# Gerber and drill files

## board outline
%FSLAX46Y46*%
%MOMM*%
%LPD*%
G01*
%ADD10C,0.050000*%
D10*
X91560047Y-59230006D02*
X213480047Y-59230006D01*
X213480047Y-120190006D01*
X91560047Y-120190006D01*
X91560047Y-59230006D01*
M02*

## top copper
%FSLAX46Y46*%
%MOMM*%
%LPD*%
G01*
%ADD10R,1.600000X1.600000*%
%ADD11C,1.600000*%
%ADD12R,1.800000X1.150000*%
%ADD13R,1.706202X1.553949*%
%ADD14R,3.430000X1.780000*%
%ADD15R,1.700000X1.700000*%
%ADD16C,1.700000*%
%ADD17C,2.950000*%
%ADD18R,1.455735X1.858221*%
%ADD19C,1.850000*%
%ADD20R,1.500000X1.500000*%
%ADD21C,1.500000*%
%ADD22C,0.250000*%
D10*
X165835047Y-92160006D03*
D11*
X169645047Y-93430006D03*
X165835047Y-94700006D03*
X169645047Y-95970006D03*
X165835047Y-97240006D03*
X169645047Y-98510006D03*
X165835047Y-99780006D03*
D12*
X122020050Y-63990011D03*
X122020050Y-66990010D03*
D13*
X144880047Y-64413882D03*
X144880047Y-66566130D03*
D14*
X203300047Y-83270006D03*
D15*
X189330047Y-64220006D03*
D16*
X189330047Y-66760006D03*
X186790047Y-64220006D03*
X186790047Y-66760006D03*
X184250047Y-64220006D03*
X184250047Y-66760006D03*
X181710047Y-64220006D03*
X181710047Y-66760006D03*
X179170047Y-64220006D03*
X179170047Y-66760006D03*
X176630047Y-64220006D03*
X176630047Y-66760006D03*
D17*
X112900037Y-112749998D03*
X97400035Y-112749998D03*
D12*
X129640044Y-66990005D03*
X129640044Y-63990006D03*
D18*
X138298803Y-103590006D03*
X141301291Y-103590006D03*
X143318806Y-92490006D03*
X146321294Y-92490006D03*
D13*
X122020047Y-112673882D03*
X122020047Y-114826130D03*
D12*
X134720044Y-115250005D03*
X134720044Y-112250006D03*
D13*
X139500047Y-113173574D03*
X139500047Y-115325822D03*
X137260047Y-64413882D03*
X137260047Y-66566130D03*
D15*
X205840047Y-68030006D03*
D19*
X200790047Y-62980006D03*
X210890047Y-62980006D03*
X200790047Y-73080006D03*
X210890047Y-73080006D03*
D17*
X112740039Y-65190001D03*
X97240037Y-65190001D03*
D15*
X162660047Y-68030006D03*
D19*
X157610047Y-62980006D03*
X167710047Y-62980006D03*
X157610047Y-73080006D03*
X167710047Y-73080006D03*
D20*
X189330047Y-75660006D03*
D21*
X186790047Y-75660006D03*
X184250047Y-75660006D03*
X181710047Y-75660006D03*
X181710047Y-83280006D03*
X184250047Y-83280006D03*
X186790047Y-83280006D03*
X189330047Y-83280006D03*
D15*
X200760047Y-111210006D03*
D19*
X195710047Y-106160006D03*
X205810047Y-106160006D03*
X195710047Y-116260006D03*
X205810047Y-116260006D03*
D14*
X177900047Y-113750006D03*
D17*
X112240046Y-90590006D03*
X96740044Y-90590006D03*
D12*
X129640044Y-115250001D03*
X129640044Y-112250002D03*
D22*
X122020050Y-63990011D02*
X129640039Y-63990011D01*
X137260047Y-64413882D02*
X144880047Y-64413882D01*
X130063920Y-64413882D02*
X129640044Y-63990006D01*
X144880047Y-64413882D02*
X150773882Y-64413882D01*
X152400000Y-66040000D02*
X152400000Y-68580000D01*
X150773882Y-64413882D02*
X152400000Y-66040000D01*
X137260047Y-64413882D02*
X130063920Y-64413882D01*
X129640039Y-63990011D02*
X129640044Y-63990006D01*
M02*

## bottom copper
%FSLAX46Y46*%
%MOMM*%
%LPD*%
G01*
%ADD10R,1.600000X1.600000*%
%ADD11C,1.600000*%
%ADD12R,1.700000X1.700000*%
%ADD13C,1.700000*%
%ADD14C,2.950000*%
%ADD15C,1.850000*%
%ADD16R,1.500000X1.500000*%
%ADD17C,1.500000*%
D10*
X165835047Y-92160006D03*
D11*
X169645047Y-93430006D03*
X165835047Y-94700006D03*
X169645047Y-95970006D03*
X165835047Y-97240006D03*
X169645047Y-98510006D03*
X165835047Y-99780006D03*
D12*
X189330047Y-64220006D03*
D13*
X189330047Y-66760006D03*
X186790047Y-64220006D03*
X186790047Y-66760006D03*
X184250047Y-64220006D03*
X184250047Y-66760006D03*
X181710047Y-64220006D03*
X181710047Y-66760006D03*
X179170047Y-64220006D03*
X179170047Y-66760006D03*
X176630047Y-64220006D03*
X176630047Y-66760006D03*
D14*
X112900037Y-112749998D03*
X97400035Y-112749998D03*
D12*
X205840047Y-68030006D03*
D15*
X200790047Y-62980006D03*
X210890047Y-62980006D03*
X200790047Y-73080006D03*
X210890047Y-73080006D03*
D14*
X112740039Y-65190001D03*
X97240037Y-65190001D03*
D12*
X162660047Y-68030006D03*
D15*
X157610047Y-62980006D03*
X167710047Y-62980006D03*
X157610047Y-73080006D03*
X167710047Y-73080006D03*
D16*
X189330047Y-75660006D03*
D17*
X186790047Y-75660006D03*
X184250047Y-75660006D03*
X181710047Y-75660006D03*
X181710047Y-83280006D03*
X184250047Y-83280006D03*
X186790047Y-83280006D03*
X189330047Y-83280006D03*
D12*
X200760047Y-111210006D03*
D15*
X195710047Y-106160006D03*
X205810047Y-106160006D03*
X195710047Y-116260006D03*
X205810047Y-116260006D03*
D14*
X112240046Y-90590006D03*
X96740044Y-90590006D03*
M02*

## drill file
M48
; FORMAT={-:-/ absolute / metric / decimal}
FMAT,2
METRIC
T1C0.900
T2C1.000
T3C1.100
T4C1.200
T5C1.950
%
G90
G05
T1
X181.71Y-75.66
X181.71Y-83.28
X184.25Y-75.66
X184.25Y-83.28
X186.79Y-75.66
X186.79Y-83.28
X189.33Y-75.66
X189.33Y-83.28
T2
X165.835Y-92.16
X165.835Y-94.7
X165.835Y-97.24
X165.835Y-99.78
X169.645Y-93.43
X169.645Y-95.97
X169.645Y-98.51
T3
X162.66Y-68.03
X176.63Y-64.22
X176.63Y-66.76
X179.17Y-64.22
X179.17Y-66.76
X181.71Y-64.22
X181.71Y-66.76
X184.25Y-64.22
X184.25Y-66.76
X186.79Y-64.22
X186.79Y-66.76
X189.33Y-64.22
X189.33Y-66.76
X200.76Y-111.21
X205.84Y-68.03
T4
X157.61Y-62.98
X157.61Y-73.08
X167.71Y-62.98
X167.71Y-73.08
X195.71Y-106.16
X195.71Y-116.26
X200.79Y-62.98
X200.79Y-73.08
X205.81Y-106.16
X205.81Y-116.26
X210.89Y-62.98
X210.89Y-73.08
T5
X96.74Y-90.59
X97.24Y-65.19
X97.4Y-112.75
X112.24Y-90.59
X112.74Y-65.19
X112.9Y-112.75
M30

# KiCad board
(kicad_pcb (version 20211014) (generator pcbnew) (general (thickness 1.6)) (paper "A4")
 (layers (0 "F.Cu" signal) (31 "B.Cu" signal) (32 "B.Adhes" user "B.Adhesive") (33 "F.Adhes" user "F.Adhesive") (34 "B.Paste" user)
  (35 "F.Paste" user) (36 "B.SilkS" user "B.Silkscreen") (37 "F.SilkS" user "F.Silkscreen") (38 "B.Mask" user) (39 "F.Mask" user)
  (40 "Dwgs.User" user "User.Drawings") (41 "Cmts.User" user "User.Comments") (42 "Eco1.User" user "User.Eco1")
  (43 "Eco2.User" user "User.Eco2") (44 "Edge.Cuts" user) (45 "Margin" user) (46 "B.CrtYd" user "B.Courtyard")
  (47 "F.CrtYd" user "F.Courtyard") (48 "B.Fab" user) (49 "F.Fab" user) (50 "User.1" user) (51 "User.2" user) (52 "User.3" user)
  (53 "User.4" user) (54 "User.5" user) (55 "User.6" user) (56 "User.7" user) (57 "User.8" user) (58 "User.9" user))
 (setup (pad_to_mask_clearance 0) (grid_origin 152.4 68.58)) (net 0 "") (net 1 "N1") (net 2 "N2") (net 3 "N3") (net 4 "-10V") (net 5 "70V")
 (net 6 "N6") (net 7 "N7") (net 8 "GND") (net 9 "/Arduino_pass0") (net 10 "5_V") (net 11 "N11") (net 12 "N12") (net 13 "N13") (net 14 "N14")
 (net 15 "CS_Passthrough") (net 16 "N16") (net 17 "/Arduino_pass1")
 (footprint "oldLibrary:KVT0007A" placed (layer "F.Cu") (at 167.740047 95.970006)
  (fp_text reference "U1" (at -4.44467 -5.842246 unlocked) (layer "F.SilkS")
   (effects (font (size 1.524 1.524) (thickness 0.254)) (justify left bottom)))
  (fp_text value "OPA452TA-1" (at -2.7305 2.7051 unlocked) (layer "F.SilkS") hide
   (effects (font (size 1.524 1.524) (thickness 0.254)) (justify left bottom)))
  (pad "1" thru_hole rect (at -1.905 -3.81) (size 1.6 1.6) (drill 1) (layers *.Cu *.Mask) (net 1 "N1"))
  (pad "2" thru_hole circle (at 1.905 -2.54) (size 1.6 1.6) (drill 1) (layers *.Cu *.Mask) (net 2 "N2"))
  (pad "3" thru_hole circle (at -1.905 -1.27) (size 1.6 1.6) (drill 1) (layers *.Cu *.Mask) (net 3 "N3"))
  (pad "4" thru_hole circle (at 1.905 0) (size 1.6 1.6) (drill 1) (layers *.Cu *.Mask) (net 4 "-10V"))
  (pad "5" thru_hole circle (at -1.905 1.27) (size 1.6 1.6) (drill 1) (layers *.Cu *.Mask) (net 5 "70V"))
  (pad "6" thru_hole circle (at 1.905 2.54) (size 1.6 1.6) (drill 1) (layers *.Cu *.Mask) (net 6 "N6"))
  (pad "7" thru_hole circle (at -1.905 3.81) (size 1.6 1.6) (drill 1) (layers *.Cu *.Mask) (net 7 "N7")))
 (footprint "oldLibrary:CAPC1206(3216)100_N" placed (layer "F.Cu") (at 122.020047 65.49001 -90)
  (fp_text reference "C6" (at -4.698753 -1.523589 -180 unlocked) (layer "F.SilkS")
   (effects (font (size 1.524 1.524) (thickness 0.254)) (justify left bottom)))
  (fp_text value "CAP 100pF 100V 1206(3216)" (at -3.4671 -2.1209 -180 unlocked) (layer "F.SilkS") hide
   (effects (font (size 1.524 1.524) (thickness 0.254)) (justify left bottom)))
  (pad "1" smd rect (at -1.499999 -0.000003) (size 1.8 1.15) (layers "F.Cu" "F.Paste" "F.Mask") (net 4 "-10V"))
  (pad "2" smd rect (at 1.5 -0.000003) (size 1.8 1.15) (layers "F.Cu" "F.Paste" "F.Mask") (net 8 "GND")))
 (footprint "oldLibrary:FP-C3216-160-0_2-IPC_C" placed (layer "F.Cu") (at 144.880047 65.490006 -90)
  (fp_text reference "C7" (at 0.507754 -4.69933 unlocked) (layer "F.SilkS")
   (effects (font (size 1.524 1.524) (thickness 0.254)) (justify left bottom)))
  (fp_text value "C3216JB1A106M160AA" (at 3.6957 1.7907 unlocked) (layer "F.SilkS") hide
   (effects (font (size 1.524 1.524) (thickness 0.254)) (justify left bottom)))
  (pad "1" smd rect (at -1.076124 0 270) (size 1.553949 1.706202) (layers "F.Cu" "F.Paste" "F.Mask") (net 4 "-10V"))
  (pad "2" smd rect (at 1.076124 0 270) (size 1.553949 1.706202) (layers "F.Cu" "F.Paste" "F.Mask") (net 8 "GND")))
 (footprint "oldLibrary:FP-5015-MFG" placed (layer "F.Cu") (at 203.300047 83.270006)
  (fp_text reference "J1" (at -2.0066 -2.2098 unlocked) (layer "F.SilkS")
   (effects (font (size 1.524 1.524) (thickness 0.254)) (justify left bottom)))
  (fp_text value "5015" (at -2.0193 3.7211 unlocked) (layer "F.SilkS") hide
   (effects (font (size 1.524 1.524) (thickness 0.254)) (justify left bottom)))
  (pad "1" smd rect (at 0 0) (size 3.43 1.78) (layers "F.Cu" "F.Paste" "F.Mask") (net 2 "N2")))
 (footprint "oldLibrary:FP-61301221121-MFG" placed (layer "F.Cu") (at 182.980047 65.490006 180)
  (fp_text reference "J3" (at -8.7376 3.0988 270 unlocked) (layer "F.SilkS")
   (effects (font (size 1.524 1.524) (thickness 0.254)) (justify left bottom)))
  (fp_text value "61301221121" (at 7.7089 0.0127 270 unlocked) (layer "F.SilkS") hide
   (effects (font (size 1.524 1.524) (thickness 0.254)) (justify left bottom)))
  (pad "1" thru_hole rect (at -6.35 1.27 180) (size 1.7 1.7) (drill 1.1) (layers *.Cu *.Mask) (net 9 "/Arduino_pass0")
   (solder_paste_margin -1000))
  (pad "2" thru_hole circle (at -6.35 -1.27 180) (size 1.7 1.7) (drill 1.1) (layers *.Cu *.Mask) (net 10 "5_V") (solder_paste_margin -1000))
  (pad "3" thru_hole circle (at -3.81 1.27 180) (size 1.7 1.7) (drill 1.1) (layers *.Cu *.Mask) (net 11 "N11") (solder_paste_margin -1000))
  (pad "4" thru_hole circle (at -3.81 -1.27 180) (size 1.7 1.7) (drill 1.1) (layers *.Cu *.Mask) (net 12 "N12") (solder_paste_margin -1000))
  (pad "5" thru_hole circle (at -1.27 1.27 180) (size 1.7 1.7) (drill 1.1) (layers *.Cu *.Mask) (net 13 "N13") (solder_paste_margin -1000))
  (pad "6" thru_hole circle (at -1.27 -1.27 180) (size 1.7 1.7) (drill 1.1) (layers *.Cu *.Mask) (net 13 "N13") (solder_paste_margin -1000))
  (pad "7" thru_hole circle (at 1.27 1.27 180) (size 1.7 1.7) (drill 1.1) (layers *.Cu *.Mask) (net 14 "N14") (solder_paste_margin -1000))
  (pad "8" thru_hole circle (at 1.27 -1.27 180) (size 1.7 1.7) (drill 1.1) (layers *.Cu *.Mask) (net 14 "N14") (solder_paste_margin -1000))
  (pad "9" thru_hole circle (at 3.81 1.27 180) (size 1.7 1.7) (drill 1.1) (layers *.Cu *.Mask) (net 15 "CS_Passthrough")
   (solder_paste_margin -1000))
  (pad "10" thru_hole circle (at 3.81 -1.27 180) (size 1.7 1.7) (drill 1.1) (layers *.Cu *.Mask) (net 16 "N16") (solder_paste_margin -1000))
  (pad "11" thru_hole circle (at 6.35 1.27 180) (size 1.7 1.7) (drill 1.1) (layers *.Cu *.Mask) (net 15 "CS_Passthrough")
   (solder_paste_margin -1000))
  (pad "12" thru_hole circle (at 6.35 -1.27 180) (size 1.7 1.7) (drill 1.1) (layers *.Cu *.Mask) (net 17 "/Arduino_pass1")
   (solder_paste_margin -1000)))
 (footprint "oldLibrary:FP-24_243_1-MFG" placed (layer "F.Cu") (at 104.400037 113.049998)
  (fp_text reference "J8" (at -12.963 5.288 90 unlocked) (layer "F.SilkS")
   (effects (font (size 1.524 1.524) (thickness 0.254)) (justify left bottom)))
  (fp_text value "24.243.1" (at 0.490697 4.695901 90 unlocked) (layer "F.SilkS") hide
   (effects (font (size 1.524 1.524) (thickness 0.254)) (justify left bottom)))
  (pad "1" thru_hole circle (at 8.5 -0.3) (size 2.95 2.95) (drill 1.95) (layers *.Cu *.Mask) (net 8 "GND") (solder_paste_margin -1000))
  (pad "1" thru_hole circle (at -7.000002 -0.3) (size 2.95 2.95) (drill 1.95) (layers *.Cu *.Mask) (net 8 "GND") (solder_paste_margin -1000)))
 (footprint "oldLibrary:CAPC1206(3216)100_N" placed (layer "F.Cu") (at 129.640047 65.490006 90)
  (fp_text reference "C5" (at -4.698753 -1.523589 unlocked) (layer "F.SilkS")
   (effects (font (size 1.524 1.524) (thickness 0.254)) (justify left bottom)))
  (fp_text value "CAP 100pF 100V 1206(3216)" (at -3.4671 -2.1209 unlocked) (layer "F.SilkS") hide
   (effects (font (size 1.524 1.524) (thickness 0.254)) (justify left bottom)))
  (pad "1" smd rect (at -1.499999 -0.000003 180) (size 1.8 1.15) (layers "F.Cu" "F.Paste" "F.Mask") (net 8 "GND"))
  (pad "2" smd rect (at 1.5 -0.000003 180) (size 1.8 1.15) (layers "F.Cu" "F.Paste" "F.Mask") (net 4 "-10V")))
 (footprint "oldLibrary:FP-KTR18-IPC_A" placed (layer "F.Cu") (at 139.800047 103.590006)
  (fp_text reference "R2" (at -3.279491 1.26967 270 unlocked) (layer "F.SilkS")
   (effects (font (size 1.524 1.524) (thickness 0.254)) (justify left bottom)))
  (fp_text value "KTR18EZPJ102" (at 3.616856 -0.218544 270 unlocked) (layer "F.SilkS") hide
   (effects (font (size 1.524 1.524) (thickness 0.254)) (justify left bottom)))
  (pad "1" smd rect (at -1.501244 0 180) (size 1.455735 1.858221) (layers "F.Cu" "F.Paste" "F.Mask") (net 8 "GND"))
  (pad "2" smd rect (at 1.501244 0 180) (size 1.455735 1.858221) (layers "F.Cu" "F.Paste" "F.Mask") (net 1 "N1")))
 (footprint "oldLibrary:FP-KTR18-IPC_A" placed (layer "F.Cu") (at 144.82005 92.490006)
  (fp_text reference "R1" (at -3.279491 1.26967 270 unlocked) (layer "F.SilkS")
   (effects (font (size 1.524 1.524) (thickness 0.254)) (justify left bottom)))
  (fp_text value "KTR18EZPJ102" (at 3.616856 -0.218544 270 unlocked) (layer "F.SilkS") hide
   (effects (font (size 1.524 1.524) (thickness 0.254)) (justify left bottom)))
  (pad "1" smd rect (at -1.501244 0 180) (size 1.455735 1.858221) (layers "F.Cu" "F.Paste" "F.Mask") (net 1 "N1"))
  (pad "2" smd rect (at 1.501244 0 180) (size 1.455735 1.858221) (layers "F.Cu" "F.Paste" "F.Mask") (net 6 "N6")))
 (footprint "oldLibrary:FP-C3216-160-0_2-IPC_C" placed (layer "F.Cu") (at 122.020047 113.750006 -90)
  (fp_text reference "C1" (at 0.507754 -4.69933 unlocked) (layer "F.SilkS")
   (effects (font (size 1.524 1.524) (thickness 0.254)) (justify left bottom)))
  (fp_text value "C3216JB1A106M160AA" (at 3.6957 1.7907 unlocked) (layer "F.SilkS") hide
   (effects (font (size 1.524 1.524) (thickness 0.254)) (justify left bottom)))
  (pad "1" smd rect (at -1.076124 0 270) (size 1.553949 1.706202) (layers "F.Cu" "F.Paste" "F.Mask") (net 5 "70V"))
  (pad "2" smd rect (at 1.076124 0 270) (size 1.553949 1.706202) (layers "F.Cu" "F.Paste" "F.Mask") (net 8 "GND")))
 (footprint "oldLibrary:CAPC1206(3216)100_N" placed (layer "F.Cu") (at 134.720047 113.750006 90)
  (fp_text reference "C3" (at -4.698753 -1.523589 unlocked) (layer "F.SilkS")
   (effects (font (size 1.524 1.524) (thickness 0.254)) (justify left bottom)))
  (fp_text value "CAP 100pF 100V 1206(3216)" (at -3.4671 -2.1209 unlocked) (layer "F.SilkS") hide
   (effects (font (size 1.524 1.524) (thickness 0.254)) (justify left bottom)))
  (pad "1" smd rect (at -1.499999 -0.000003 180) (size 1.8 1.15) (layers "F.Cu" "F.Paste" "F.Mask") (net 8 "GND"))
  (pad "2" smd rect (at 1.5 -0.000003 180) (size 1.8 1.15) (layers "F.Cu" "F.Paste" "F.Mask") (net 5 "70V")))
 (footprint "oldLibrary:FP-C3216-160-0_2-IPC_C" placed (layer "F.Cu") (at 139.500047 114.249698 -90)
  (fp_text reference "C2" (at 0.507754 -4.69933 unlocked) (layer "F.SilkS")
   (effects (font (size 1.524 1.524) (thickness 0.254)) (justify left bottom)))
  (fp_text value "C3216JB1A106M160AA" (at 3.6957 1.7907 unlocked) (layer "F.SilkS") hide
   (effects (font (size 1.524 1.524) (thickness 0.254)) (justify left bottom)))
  (pad "1" smd rect (at -1.076124 0 270) (size 1.553949 1.706202) (layers "F.Cu" "F.Paste" "F.Mask") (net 5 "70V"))
  (pad "2" smd rect (at 1.076124 0 270) (size 1.553949 1.706202) (layers "F.Cu" "F.Paste" "F.Mask") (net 8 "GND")))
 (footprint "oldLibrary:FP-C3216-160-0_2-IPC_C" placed (layer "F.Cu") (at 137.260047 65.490006 -90)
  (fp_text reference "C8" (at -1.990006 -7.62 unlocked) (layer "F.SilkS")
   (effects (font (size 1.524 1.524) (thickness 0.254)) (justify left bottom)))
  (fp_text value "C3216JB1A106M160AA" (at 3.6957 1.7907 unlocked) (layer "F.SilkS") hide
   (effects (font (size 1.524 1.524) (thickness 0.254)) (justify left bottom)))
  (pad "1" smd rect (at -1.076124 0 270) (size 1.553949 1.706202) (layers "F.Cu" "F.Paste" "F.Mask") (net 4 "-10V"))
  (pad "2" smd rect (at 1.076124 0 270) (size 1.553949 1.706202) (layers "F.Cu" "F.Paste" "F.Mask") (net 8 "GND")))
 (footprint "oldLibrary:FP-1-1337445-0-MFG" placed (layer "F.Cu") (at 205.840047 68.030006)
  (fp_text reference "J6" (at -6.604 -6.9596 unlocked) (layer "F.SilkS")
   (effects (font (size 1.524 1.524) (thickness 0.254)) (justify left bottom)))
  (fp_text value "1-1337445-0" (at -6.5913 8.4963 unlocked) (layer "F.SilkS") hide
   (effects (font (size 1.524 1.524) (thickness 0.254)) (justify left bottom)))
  (pad "1" thru_hole rect (at 0 0) (size 1.7 1.7) (drill 1.1) (layers *.Cu *.Mask) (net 9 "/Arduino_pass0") (solder_paste_margin -1000))
  (pad "2" thru_hole circle (at -5.05 -5.05) (size 1.85 1.85) (drill 1.2) (layers *.Cu *.Mask) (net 8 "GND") (solder_paste_margin -1000))
  (pad "3" thru_hole circle (at 5.05 -5.05) (size 1.85 1.85) (drill 1.2) (layers *.Cu *.Mask) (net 8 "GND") (solder_paste_margin -1000))
  (pad "4" thru_hole circle (at -5.05 5.05) (size 1.85 1.85) (drill 1.2) (layers *.Cu *.Mask) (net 8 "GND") (solder_paste_margin -1000))
  (pad "5" thru_hole circle (at 5.05 5.05) (size 1.85 1.85) (drill 1.2) (layers *.Cu *.Mask) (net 8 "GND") (solder_paste_margin -1000)))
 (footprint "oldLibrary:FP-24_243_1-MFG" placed (layer "F.Cu") (at 104.240039 65.490001)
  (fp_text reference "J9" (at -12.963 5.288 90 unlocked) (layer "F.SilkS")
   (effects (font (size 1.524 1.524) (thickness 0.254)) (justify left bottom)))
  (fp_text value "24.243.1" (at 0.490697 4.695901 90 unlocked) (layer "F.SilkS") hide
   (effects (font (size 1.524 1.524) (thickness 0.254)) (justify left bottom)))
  (pad "1" thru_hole circle (at 8.5 -0.3) (size 2.95 2.95) (drill 1.95) (layers *.Cu *.Mask) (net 4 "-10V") (solder_paste_margin -1000))
  (pad "1" thru_hole circle (at -7.000002 -0.3) (size 2.95 2.95) (drill 1.95) (layers *.Cu *.Mask) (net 4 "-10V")
   (solder_paste_margin -1000)))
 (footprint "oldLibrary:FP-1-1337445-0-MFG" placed (layer "F.Cu") (at 162.660047 68.030006)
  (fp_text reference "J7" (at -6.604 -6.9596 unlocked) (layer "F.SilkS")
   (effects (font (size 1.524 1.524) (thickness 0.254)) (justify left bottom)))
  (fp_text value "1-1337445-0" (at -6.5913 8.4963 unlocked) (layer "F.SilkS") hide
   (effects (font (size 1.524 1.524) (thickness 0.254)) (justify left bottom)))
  (pad "1" thru_hole rect (at 0 0) (size 1.7 1.7) (drill 1.1) (layers *.Cu *.Mask) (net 17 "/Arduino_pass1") (solder_paste_margin -1000))
  (pad "2" thru_hole circle (at -5.05 -5.05) (size 1.85 1.85) (drill 1.2) (layers *.Cu *.Mask) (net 8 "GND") (solder_paste_margin -1000))
  (pad "3" thru_hole circle (at 5.05 -5.05) (size 1.85 1.85) (drill 1.2) (layers *.Cu *.Mask) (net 8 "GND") (solder_paste_margin -1000))
  (pad "4" thru_hole circle (at -5.05 5.05) (size 1.85 1.85) (drill 1.2) (layers *.Cu *.Mask) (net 8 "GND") (solder_paste_margin -1000))
  (pad "5" thru_hole circle (at 5.05 5.05) (size 1.85 1.85) (drill 1.2) (layers *.Cu *.Mask) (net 8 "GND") (solder_paste_margin -1000)))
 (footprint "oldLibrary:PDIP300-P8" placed (layer "F.Cu") (at 185.520047 79.470006 -90)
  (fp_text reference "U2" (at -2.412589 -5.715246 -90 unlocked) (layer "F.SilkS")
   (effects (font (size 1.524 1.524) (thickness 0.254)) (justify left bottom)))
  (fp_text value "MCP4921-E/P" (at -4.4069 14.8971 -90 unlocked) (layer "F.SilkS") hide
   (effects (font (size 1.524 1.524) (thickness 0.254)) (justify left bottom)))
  (pad "1" thru_hole rect (at -3.81 -3.81 270) (size 1.5 1.5) (drill 0.9) (layers *.Cu *.Mask) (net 10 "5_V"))
  (pad "2" thru_hole circle (at -3.81 -1.27 270) (size 1.5 1.5) (drill 0.9) (layers *.Cu *.Mask) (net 12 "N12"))
  (pad "3" thru_hole circle (at -3.81 1.27 270) (size 1.5 1.5) (drill 0.9) (layers *.Cu *.Mask) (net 13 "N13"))
  (pad "4" thru_hole circle (at -3.81 3.81 270) (size 1.5 1.5) (drill 0.9) (layers *.Cu *.Mask) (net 14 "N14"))
  (pad "5" thru_hole circle (at 3.81 3.81 270) (size 1.5 1.5) (drill 0.9) (layers *.Cu *.Mask) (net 16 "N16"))
  (pad "6" thru_hole circle (at 3.81 1.27 270) (size 1.5 1.5) (drill 0.9) (layers *.Cu *.Mask) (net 10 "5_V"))
  (pad "7" thru_hole circle (at 3.81 -1.27 270) (size 1.5 1.5) (drill 0.9) (layers *.Cu *.Mask) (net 8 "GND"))
  (pad "8" thru_hole circle (at 3.81 -3.81 270) (size 1.5 1.5) (drill 0.9) (layers *.Cu *.Mask) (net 2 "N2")))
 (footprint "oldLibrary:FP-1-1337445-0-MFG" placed (layer "F.Cu") (at 200.760047 111.210006)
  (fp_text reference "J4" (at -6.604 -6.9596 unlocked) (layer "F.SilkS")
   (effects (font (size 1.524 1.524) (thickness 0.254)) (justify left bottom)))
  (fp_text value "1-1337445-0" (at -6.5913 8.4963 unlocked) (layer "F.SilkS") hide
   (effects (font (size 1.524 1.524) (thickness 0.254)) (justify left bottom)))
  (pad "1" thru_hole rect (at 0 0) (size 1.7 1.7) (drill 1.1) (layers *.Cu *.Mask) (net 6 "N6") (solder_paste_margin -1000))
  (pad "2" thru_hole circle (at -5.05 -5.05) (size 1.85 1.85) (drill 1.2) (layers *.Cu *.Mask) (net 8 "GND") (solder_paste_margin -1000))
  (pad "3" thru_hole circle (at 5.05 -5.05) (size 1.85 1.85) (drill 1.2) (layers *.Cu *.Mask) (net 8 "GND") (solder_paste_margin -1000))
  (pad "4" thru_hole circle (at -5.05 5.05) (size 1.85 1.85) (drill 1.2) (layers *.Cu *.Mask) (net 8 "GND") (solder_paste_margin -1000))
  (pad "5" thru_hole circle (at 5.05 5.05) (size 1.85 1.85) (drill 1.2) (layers *.Cu *.Mask) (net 8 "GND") (solder_paste_margin -1000)))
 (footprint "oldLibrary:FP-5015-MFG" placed (layer "F.Cu") (at 177.900047 113.750006)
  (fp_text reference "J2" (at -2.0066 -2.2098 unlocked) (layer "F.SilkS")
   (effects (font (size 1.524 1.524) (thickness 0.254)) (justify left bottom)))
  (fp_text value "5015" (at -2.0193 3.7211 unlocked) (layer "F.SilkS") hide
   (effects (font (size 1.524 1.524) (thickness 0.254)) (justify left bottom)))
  (pad "1" smd rect (at 0 0) (size 3.43 1.78) (layers "F.Cu" "F.Paste" "F.Mask") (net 6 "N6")))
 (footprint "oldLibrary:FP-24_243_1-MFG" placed (layer "F.Cu") (at 103.740046 90.890006)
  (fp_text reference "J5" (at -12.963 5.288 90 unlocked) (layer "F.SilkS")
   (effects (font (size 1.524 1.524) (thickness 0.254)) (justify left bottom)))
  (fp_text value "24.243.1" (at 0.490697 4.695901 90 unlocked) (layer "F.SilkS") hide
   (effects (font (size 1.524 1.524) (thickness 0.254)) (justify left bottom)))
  (pad "1" thru_hole circle (at 8.5 -0.3) (size 2.95 2.95) (drill 1.95) (layers *.Cu *.Mask) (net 5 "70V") (solder_paste_margin -1000))
  (pad "1" thru_hole circle (at -7.000002 -0.3) (size 2.95 2.95) (drill 1.95) (layers *.Cu *.Mask) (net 5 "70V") (solder_paste_margin -1000)))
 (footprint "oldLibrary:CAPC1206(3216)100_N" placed (layer "F.Cu") (at 129.640047 113.750002 90)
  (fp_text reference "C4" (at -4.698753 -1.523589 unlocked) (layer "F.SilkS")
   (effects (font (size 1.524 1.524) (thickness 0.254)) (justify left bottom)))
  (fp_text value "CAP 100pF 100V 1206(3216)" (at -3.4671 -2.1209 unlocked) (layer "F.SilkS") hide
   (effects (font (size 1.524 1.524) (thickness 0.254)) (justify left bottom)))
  (pad "1" smd rect (at -1.499999 -0.000003 180) (size 1.8 1.15) (layers "F.Cu" "F.Paste" "F.Mask") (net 8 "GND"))
  (pad "2" smd rect (at 1.5 -0.000003 180) (size 1.8 1.15) (layers "F.Cu" "F.Paste" "F.Mask") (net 5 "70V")))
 (gr_rect (start 213.480047 120.190006) (end 91.560047 59.230006) (layer "Edge.Cuts") (width 0.05) (fill none))
 (segment (start 122.02005 63.990011) (end 129.640039 63.990011) (width 0.25) (layer "F.Cu") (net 4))
 (segment (start 137.260047 64.413882) (end 144.880047 64.413882) (width 0.25) (layer "F.Cu") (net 4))
 (segment (start 130.06392 64.413882) (end 129.640044 63.990006) (width 0.25) (layer "F.Cu") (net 4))
 (segment (start 144.880047 64.413882) (end 150.773882 64.413882) (width 0.25) (layer "F.Cu") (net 4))
 (segment (start 152.4 66.04) (end 152.4 68.58) (width 0.25) (layer "F.Cu") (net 4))
 (segment (start 150.773882 64.413882) (end 152.4 66.04) (width 0.25) (layer "F.Cu") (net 4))
 (segment (start 137.260047 64.413882) (end 130.06392 64.413882) (width 0.25) (layer "F.Cu") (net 4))
 (segment (start 129.640039 63.990011) (end 129.640044 63.990006) (width 0.25) (layer "F.Cu") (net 4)))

